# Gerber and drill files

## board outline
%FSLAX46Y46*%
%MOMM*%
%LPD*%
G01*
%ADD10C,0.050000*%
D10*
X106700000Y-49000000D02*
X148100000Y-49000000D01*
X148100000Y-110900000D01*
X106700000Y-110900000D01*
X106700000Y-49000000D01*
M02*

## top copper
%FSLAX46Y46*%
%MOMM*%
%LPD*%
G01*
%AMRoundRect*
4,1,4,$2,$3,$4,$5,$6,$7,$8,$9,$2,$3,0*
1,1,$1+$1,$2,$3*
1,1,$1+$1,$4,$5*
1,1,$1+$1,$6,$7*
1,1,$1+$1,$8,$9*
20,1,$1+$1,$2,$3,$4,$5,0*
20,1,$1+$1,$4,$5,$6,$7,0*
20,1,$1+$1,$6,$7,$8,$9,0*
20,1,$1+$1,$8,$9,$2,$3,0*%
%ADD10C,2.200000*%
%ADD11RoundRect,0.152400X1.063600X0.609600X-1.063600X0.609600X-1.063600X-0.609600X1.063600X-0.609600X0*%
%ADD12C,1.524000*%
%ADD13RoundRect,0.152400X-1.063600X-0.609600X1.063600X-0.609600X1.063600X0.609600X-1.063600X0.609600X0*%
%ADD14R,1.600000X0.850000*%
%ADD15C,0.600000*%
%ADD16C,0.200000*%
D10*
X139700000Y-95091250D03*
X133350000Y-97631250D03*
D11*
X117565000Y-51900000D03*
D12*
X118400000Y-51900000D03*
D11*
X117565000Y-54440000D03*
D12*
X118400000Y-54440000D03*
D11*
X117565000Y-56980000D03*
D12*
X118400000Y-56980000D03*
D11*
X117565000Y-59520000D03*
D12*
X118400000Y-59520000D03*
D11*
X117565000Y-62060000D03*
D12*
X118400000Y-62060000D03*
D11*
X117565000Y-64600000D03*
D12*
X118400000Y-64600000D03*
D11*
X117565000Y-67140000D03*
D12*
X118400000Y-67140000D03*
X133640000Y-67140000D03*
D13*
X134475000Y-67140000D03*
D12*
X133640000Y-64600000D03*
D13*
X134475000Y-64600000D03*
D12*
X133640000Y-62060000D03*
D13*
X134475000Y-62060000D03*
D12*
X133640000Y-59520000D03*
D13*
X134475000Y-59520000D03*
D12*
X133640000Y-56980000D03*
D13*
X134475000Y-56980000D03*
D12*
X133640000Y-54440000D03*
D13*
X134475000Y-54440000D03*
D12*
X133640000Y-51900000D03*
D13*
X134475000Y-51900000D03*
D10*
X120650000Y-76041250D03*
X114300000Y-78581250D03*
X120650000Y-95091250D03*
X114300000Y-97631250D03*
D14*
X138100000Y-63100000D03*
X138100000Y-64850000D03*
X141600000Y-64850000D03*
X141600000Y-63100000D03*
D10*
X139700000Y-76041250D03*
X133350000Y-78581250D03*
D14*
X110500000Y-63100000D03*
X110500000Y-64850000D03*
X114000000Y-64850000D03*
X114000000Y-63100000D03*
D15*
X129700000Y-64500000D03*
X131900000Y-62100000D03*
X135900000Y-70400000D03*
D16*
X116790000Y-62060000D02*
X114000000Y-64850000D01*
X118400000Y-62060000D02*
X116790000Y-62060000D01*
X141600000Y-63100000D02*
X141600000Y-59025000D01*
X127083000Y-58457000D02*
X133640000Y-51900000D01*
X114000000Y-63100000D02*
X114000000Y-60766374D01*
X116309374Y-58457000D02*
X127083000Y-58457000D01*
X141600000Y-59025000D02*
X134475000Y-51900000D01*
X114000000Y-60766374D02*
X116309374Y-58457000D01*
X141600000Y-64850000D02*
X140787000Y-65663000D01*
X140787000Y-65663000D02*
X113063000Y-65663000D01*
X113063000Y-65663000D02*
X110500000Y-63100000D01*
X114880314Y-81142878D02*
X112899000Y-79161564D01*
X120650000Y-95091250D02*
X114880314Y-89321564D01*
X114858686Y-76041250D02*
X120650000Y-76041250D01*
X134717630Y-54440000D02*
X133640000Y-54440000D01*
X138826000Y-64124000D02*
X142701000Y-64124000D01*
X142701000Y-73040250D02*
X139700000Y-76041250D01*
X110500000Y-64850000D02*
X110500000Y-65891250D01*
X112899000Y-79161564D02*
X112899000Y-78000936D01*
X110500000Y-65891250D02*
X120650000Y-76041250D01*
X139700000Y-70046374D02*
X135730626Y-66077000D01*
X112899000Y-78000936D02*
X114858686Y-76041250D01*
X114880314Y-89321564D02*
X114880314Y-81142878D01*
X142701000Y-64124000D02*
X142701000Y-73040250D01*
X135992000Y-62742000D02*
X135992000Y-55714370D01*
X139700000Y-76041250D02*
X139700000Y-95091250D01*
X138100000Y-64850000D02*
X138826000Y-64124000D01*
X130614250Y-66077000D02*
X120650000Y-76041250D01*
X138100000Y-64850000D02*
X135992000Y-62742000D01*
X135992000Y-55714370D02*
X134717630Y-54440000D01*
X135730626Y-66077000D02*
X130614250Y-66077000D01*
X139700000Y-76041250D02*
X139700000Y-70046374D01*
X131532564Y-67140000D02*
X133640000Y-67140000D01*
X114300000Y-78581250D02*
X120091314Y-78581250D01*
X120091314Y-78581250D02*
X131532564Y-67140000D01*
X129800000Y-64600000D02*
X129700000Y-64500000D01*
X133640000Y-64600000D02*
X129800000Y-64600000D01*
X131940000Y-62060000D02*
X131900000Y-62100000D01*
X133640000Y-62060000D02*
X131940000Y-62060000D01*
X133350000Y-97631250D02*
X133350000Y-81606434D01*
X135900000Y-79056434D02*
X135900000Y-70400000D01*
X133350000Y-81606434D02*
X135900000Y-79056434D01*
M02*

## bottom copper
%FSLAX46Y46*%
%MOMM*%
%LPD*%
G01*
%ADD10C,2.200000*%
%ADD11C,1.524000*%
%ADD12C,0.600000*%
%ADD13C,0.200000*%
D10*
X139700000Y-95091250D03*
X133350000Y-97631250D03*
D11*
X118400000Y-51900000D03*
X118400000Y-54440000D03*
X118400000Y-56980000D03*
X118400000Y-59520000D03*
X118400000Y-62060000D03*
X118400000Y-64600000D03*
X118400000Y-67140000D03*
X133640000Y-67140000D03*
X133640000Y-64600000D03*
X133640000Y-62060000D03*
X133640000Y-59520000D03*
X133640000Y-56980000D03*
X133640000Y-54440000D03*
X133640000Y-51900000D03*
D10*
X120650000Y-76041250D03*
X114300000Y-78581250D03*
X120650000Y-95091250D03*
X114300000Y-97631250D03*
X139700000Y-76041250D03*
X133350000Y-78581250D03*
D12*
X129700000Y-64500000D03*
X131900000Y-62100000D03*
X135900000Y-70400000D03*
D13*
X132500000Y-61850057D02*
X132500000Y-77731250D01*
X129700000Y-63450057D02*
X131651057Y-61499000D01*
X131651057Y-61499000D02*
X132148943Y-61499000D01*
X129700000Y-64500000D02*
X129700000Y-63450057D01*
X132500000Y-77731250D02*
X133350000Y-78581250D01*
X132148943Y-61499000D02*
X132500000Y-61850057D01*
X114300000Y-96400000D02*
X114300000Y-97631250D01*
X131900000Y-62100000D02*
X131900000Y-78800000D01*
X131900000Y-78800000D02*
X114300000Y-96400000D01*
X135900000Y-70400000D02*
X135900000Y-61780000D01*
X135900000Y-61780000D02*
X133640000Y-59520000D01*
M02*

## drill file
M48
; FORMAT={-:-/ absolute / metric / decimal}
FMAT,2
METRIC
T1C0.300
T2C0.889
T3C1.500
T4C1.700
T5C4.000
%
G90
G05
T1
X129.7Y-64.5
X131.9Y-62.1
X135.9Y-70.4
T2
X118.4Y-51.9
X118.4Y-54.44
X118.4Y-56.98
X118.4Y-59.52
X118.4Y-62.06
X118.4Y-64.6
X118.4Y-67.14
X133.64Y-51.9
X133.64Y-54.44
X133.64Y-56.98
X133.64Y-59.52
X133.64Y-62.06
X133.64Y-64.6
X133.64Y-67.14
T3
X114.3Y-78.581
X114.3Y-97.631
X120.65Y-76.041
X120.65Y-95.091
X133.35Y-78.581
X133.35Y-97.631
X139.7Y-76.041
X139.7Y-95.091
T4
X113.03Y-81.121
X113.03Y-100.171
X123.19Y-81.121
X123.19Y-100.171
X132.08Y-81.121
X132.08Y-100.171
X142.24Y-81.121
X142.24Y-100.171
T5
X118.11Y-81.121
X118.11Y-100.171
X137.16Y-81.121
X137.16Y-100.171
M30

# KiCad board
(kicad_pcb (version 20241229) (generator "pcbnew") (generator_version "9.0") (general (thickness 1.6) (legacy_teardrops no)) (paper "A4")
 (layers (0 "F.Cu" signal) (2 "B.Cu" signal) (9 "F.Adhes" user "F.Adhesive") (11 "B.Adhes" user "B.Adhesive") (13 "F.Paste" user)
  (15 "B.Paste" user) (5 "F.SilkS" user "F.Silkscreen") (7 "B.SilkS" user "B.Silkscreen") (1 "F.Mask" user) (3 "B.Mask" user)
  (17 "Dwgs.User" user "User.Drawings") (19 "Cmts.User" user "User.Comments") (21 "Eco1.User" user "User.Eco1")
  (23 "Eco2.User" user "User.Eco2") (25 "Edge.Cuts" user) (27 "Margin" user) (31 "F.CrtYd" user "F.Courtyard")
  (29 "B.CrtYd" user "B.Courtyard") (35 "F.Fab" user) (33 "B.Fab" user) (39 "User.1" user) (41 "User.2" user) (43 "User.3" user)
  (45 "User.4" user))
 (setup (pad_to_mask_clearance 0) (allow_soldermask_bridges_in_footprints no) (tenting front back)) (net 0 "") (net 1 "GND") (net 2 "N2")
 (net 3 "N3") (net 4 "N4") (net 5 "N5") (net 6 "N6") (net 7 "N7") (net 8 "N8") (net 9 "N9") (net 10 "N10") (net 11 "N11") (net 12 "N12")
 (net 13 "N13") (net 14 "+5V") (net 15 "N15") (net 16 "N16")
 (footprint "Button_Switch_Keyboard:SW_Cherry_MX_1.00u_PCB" (layer "F.Cu") (at 139.7 95.09125)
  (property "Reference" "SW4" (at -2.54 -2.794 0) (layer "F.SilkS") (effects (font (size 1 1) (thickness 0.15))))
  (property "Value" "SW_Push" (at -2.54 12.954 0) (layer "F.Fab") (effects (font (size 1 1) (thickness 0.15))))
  (pad "" np_thru_hole circle (at -7.62 5.08) (size 1.7 1.7) (drill 1.7) (layers "*.Cu" "*.Mask"))
  (pad "" np_thru_hole circle (at -2.54 5.08) (size 4 4) (drill 4) (layers "*.Cu" "*.Mask"))
  (pad "" np_thru_hole circle (at 2.54 5.08) (size 1.7 1.7) (drill 1.7) (layers "*.Cu" "*.Mask"))
  (pad "1" thru_hole circle (at 0 0) (size 2.2 2.2) (drill 1.5) (layers "*.Cu" "*.Mask") (remove_unused_layers no) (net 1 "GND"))
  (pad "2" thru_hole circle (at -6.35 2.54) (size 2.2 2.2) (drill 1.5) (layers "*.Cu" "*.Mask") (remove_unused_layers no) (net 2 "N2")))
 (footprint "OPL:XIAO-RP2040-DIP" (layer "F.Cu") (at 126.02 59.52)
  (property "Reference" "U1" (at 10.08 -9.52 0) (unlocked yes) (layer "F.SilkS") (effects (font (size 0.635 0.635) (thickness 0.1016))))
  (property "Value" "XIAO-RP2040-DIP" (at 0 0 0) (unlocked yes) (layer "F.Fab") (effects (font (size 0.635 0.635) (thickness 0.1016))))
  (pad "1" smd roundrect (at -8.455 -7.62 180) (size 2.432 1.524) (layers "F.Cu" "F.Mask") (roundrect_rratio 0.1) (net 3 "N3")
   (thermal_bridge_angle 45))
  (pad "1" thru_hole circle (at -7.62 -7.62 180) (size 1.524 1.524) (drill 0.889) (layers "*.Cu" "*.Mask") (remove_unused_layers no)
   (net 3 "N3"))
  (pad "2" smd roundrect (at -8.455 -5.08 180) (size 2.432 1.524) (layers "F.Cu" "F.Mask") (roundrect_rratio 0.1) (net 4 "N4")
   (thermal_bridge_angle 45))
  (pad "2" thru_hole circle (at -7.62 -5.08 180) (size 1.524 1.524) (drill 0.889) (layers "*.Cu" "*.Mask") (remove_unused_layers no)
   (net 4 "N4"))
  (pad "3" smd roundrect (at -8.455 -2.54 180) (size 2.432 1.524) (layers "F.Cu" "F.Mask") (roundrect_rratio 0.1) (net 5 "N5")
   (thermal_bridge_angle 45))
  (pad "3" thru_hole circle (at -7.62 -2.54 180) (size 1.524 1.524) (drill 0.889) (layers "*.Cu" "*.Mask") (remove_unused_layers no)
   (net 5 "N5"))
  (pad "4" smd roundrect (at -8.455 0 180) (size 2.432 1.524) (layers "F.Cu" "F.Mask") (roundrect_rratio 0.1) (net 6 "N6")
   (thermal_bridge_angle 45))
  (pad "4" thru_hole circle (at -7.62 0 180) (size 1.524 1.524) (drill 0.889) (layers "*.Cu" "*.Mask") (remove_unused_layers no)
   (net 6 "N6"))
  (pad "5" smd roundrect (at -8.455 2.54 180) (size 2.432 1.524) (layers "F.Cu" "F.Mask") (roundrect_rratio 0.1) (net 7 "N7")
   (thermal_bridge_angle 45))
  (pad "5" thru_hole circle (at -7.62 2.54 180) (size 1.524 1.524) (drill 0.889) (layers "*.Cu" "*.Mask") (remove_unused_layers no)
   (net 7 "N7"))
  (pad "6" smd roundrect (at -8.455 5.08 180) (size 2.432 1.524) (layers "F.Cu" "F.Mask") (roundrect_rratio 0.1) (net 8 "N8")
   (thermal_bridge_angle 45))
  (pad "6" thru_hole circle (at -7.62 5.08 180) (size 1.524 1.524) (drill 0.889) (layers "*.Cu" "*.Mask") (remove_unused_layers no)
   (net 8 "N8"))
  (pad "7" smd roundrect (at -8.455 7.62 180) (size 2.432 1.524) (layers "F.Cu" "F.Mask") (roundrect_rratio 0.1) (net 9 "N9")
   (thermal_bridge_angle 45))
  (pad "7" thru_hole circle (at -7.62 7.62 180) (size 1.524 1.524) (drill 0.889) (layers "*.Cu" "*.Mask") (remove_unused_layers no)
   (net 9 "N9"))
  (pad "8" thru_hole circle (at 7.62 7.62) (size 1.524 1.524) (drill 0.889) (layers "*.Cu" "*.Mask") (remove_unused_layers no)
   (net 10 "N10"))
  (pad "8" smd roundrect (at 8.455 7.62) (size 2.432 1.524) (layers "F.Cu" "F.Mask") (roundrect_rratio 0.1) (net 10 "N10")
   (thermal_bridge_angle 45))
  (pad "9" thru_hole circle (at 7.62 5.08) (size 1.524 1.524) (drill 0.889) (layers "*.Cu" "*.Mask") (remove_unused_layers no)
   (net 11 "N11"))
  (pad "9" smd roundrect (at 8.455 5.08) (size 2.432 1.524) (layers "F.Cu" "F.Mask") (roundrect_rratio 0.1) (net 11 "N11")
   (thermal_bridge_angle 45))
  (pad "10" thru_hole circle (at 7.62 2.54) (size 1.524 1.524) (drill 0.889) (layers "*.Cu" "*.Mask") (remove_unused_layers no)
   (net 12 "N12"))
  (pad "10" smd roundrect (at 8.455 2.54) (size 2.432 1.524) (layers "F.Cu" "F.Mask") (roundrect_rratio 0.1) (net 12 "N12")
   (thermal_bridge_angle 45))
  (pad "11" thru_hole circle (at 7.62 0) (size 1.524 1.524) (drill 0.889) (layers "*.Cu" "*.Mask") (remove_unused_layers no) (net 2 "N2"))
  (pad "11" smd roundrect (at 8.455 0) (size 2.432 1.524) (layers "F.Cu" "F.Mask") (roundrect_rratio 0.1) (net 2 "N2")
   (thermal_bridge_angle 45))
  (pad "12" thru_hole circle (at 7.62 -2.54) (size 1.524 1.524) (drill 0.889) (layers "*.Cu" "*.Mask") (remove_unused_layers no)
   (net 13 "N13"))
  (pad "12" smd roundrect (at 8.455 -2.54) (size 2.432 1.524) (layers "F.Cu" "F.Mask") (roundrect_rratio 0.1) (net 13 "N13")
   (thermal_bridge_angle 45))
  (pad "13" thru_hole circle (at 7.62 -5.08) (size 1.524 1.524) (drill 0.889) (layers "*.Cu" "*.Mask") (remove_unused_layers no)
   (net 1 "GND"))
  (pad "13" smd roundrect (at 8.455 -5.08) (size 2.432 1.524) (layers "F.Cu" "F.Mask") (roundrect_rratio 0.1) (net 1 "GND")
   (thermal_bridge_angle 45))
  (pad "14" thru_hole circle (at 7.62 -7.62) (size 1.524 1.524) (drill 0.889) (layers "*.Cu" "*.Mask") (remove_unused_layers no)
   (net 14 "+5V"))
  (pad "14" smd roundrect (at 8.455 -7.62) (size 2.432 1.524) (layers "F.Cu" "F.Mask") (roundrect_rratio 0.1) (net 14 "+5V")
   (thermal_bridge_angle 45)))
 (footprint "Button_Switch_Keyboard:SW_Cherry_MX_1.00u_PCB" (layer "F.Cu") (at 120.65 76.04125)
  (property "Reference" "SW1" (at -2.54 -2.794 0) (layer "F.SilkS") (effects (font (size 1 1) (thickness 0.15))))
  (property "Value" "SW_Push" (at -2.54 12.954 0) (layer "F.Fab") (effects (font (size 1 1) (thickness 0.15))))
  (pad "" np_thru_hole circle (at -7.62 5.08) (size 1.7 1.7) (drill 1.7) (layers "*.Cu" "*.Mask"))
  (pad "" np_thru_hole circle (at -2.54 5.08) (size 4 4) (drill 4) (layers "*.Cu" "*.Mask"))
  (pad "" np_thru_hole circle (at 2.54 5.08) (size 1.7 1.7) (drill 1.7) (layers "*.Cu" "*.Mask"))
  (pad "1" thru_hole circle (at 0 0) (size 2.2 2.2) (drill 1.5) (layers "*.Cu" "*.Mask") (remove_unused_layers no) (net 1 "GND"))
  (pad "2" thru_hole circle (at -6.35 2.54) (size 2.2 2.2) (drill 1.5) (layers "*.Cu" "*.Mask") (remove_unused_layers no) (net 10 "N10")))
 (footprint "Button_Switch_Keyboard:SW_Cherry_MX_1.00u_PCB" (layer "F.Cu") (at 120.65 95.09125)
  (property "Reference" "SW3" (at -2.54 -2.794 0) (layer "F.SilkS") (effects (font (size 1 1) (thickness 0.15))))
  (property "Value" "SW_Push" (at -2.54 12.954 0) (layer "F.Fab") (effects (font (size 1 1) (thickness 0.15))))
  (pad "" np_thru_hole circle (at -7.62 5.08) (size 1.7 1.7) (drill 1.7) (layers "*.Cu" "*.Mask"))
  (pad "" np_thru_hole circle (at -2.54 5.08) (size 4 4) (drill 4) (layers "*.Cu" "*.Mask"))
  (pad "" np_thru_hole circle (at 2.54 5.08) (size 1.7 1.7) (drill 1.7) (layers "*.Cu" "*.Mask"))
  (pad "1" thru_hole circle (at 0 0) (size 2.2 2.2) (drill 1.5) (layers "*.Cu" "*.Mask") (remove_unused_layers no) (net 1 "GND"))
  (pad "2" thru_hole circle (at -6.35 2.54) (size 2.2 2.2) (drill 1.5) (layers "*.Cu" "*.Mask") (remove_unused_layers no) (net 12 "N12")))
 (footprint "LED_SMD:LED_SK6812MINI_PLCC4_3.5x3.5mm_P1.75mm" (layer "F.Cu") (at 139.85 63.975)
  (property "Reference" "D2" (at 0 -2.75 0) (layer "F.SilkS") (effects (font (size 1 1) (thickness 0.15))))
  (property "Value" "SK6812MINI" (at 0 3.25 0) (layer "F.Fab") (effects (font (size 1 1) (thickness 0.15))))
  (pad "1" smd rect (at -1.75 -0.875) (size 1.6 0.85) (layers "F.Cu" "F.Mask" "F.Paste") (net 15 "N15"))
  (pad "2" smd rect (at -1.75 0.875) (size 1.6 0.85) (layers "F.Cu" "F.Mask" "F.Paste") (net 1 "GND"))
  (pad "3" smd rect (at 1.75 0.875) (size 1.6 0.85) (layers "F.Cu" "F.Mask" "F.Paste") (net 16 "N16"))
  (pad "4" smd rect (at 1.75 -0.875) (size 1.6 0.85) (layers "F.Cu" "F.Mask" "F.Paste") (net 14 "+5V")))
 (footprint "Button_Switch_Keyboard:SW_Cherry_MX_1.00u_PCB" (layer "F.Cu") (at 139.7 76.04125)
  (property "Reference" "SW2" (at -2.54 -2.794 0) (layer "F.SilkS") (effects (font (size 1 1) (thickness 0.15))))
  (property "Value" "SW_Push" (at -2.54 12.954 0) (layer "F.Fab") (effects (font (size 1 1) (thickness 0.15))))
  (pad "" np_thru_hole circle (at -7.62 5.08) (size 1.7 1.7) (drill 1.7) (layers "*.Cu" "*.Mask"))
  (pad "" np_thru_hole circle (at -2.54 5.08) (size 4 4) (drill 4) (layers "*.Cu" "*.Mask"))
  (pad "" np_thru_hole circle (at 2.54 5.08) (size 1.7 1.7) (drill 1.7) (layers "*.Cu" "*.Mask"))
  (pad "1" thru_hole circle (at 0 0) (size 2.2 2.2) (drill 1.5) (layers "*.Cu" "*.Mask") (remove_unused_layers no) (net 1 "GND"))
  (pad "2" thru_hole circle (at -6.35 2.54) (size 2.2 2.2) (drill 1.5) (layers "*.Cu" "*.Mask") (remove_unused_layers no) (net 11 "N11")))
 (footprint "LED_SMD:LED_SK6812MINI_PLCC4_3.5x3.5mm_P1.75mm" (layer "F.Cu") (at 112.25 63.975)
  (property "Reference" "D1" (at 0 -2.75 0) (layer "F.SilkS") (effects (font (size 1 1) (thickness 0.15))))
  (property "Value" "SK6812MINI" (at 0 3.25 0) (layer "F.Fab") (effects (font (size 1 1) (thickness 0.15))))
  (pad "1" smd rect (at -1.75 -0.875) (size 1.6 0.85) (layers "F.Cu" "F.Mask" "F.Paste") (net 16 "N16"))
  (pad "2" smd rect (at -1.75 0.875) (size 1.6 0.85) (layers "F.Cu" "F.Mask" "F.Paste") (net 1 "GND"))
  (pad "3" smd rect (at 1.75 0.875) (size 1.6 0.85) (layers "F.Cu" "F.Mask" "F.Paste") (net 7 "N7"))
  (pad "4" smd rect (at 1.75 -0.875) (size 1.6 0.85) (layers "F.Cu" "F.Mask" "F.Paste") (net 14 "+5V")))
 (gr_rect (start 106.7 49) (end 148.1 110.9) (stroke (width 0.05) (type default)) (fill no) (layer "Edge.Cuts"))
 (segment (start 116.79 62.06) (end 114 64.85) (width 0.2) (layer "F.Cu") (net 7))
 (segment (start 118.4 62.06) (end 116.79 62.06) (width 0.2) (layer "F.Cu") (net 7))
 (segment (start 141.6 63.1) (end 141.6 59.025) (width 0.2) (layer "F.Cu") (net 14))
 (segment (start 127.083 58.457) (end 133.64 51.9) (width 0.2) (layer "F.Cu") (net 14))
 (segment (start 114 63.1) (end 114 60.766374) (width 0.2) (layer "F.Cu") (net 14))
 (segment (start 116.309374 58.457) (end 127.083 58.457) (width 0.2) (layer "F.Cu") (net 14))
 (segment (start 141.6 59.025) (end 134.475 51.9) (width 0.2) (layer "F.Cu") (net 14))
 (segment (start 114 60.766374) (end 116.309374 58.457) (width 0.2) (layer "F.Cu") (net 14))
 (segment (start 141.6 64.85) (end 140.787 65.663) (width 0.2) (layer "F.Cu") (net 16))
 (segment (start 140.787 65.663) (end 113.063 65.663) (width 0.2) (layer "F.Cu") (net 16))
 (segment (start 113.063 65.663) (end 110.5 63.1) (width 0.2) (layer "F.Cu") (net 16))
 (segment (start 114.880314 81.142878) (end 112.899 79.161564) (width 0.2) (layer "F.Cu") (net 1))
 (segment (start 120.65 95.09125) (end 114.880314 89.321564) (width 0.2) (layer "F.Cu") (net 1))
 (segment (start 114.858686 76.04125) (end 120.65 76.04125) (width 0.2) (layer "F.Cu") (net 1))
 (segment (start 134.71763 54.44) (end 133.64 54.44) (width 0.2) (layer "F.Cu") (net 1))
 (segment (start 138.826 64.124) (end 142.701 64.124) (width 0.2) (layer "F.Cu") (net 1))
 (segment (start 142.701 73.04025) (end 139.7 76.04125) (width 0.2) (layer "F.Cu") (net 1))
 (segment (start 110.5 64.85) (end 110.5 65.89125) (width 0.2) (layer "F.Cu") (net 1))
 (segment (start 112.899 79.161564) (end 112.899 78.000936) (width 0.2) (layer "F.Cu") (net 1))
 (segment (start 110.5 65.89125) (end 120.65 76.04125) (width 0.2) (layer "F.Cu") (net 1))
 (segment (start 139.7 70.046374) (end 135.730626 66.077) (width 0.2) (layer "F.Cu") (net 1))
 (segment (start 112.899 78.000936) (end 114.858686 76.04125) (width 0.2) (layer "F.Cu") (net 1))
 (segment (start 114.880314 89.321564) (end 114.880314 81.142878) (width 0.2) (layer "F.Cu") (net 1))
 (segment (start 142.701 64.124) (end 142.701 73.04025) (width 0.2) (layer "F.Cu") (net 1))
 (segment (start 135.992 62.742) (end 135.992 55.71437) (width 0.2) (layer "F.Cu") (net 1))
 (segment (start 139.7 76.04125) (end 139.7 95.09125) (width 0.2) (layer "F.Cu") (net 1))
 (segment (start 138.1 64.85) (end 138.826 64.124) (width 0.2) (layer "F.Cu") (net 1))
 (segment (start 130.61425 66.077) (end 120.65 76.04125) (width 0.2) (layer "F.Cu") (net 1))
 (segment (start 138.1 64.85) (end 135.992 62.742) (width 0.2) (layer "F.Cu") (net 1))
 (segment (start 135.992 55.71437) (end 134.71763 54.44) (width 0.2) (layer "F.Cu") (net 1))
 (segment (start 135.730626 66.077) (end 130.61425 66.077) (width 0.2) (layer "F.Cu") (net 1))
 (segment (start 139.7 76.04125) (end 139.7 70.046374) (width 0.2) (layer "F.Cu") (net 1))
 (segment (start 131.532564 67.14) (end 133.64 67.14) (width 0.2) (layer "F.Cu") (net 10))
 (segment (start 114.3 78.58125) (end 120.091314 78.58125) (width 0.2) (layer "F.Cu") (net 10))
 (segment (start 120.091314 78.58125) (end 131.532564 67.14) (width 0.2) (layer "F.Cu") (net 10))
 (segment (start 129.8 64.6) (end 129.7 64.5) (width 0.2) (layer "F.Cu") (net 11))
 (segment (start 133.64 64.6) (end 129.8 64.6) (width 0.2) (layer "F.Cu") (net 11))
 (via (at 129.7 64.5) (size 0.6) (drill 0.3) (layers "F.Cu" "B.Cu") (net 11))
 (segment (start 132.5 61.850057) (end 132.5 77.73125) (width 0.2) (layer "B.Cu") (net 11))
 (segment (start 129.7 63.450057) (end 131.651057 61.499) (width 0.2) (layer "B.Cu") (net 11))
 (segment (start 131.651057 61.499) (end 132.148943 61.499) (width 0.2) (layer "B.Cu") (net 11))
 (segment (start 129.7 64.5) (end 129.7 63.450057) (width 0.2) (layer "B.Cu") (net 11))
 (segment (start 132.5 77.73125) (end 133.35 78.58125) (width 0.2) (layer "B.Cu") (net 11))
 (segment (start 132.148943 61.499) (end 132.5 61.850057) (width 0.2) (layer "B.Cu") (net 11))
 (segment (start 131.94 62.06) (end 131.9 62.1) (width 0.2) (layer "F.Cu") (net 12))
 (segment (start 133.64 62.06) (end 131.94 62.06) (width 0.2) (layer "F.Cu") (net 12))
 (via (at 131.9 62.1) (size 0.6) (drill 0.3) (layers "F.Cu" "B.Cu") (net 12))
 (segment (start 114.3 96.4) (end 114.3 97.63125) (width 0.2) (layer "B.Cu") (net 12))
 (segment (start 131.9 62.1) (end 131.9 78.8) (width 0.2) (layer "B.Cu") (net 12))
 (segment (start 131.9 78.8) (end 114.3 96.4) (width 0.2) (layer "B.Cu") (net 12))
 (segment (start 133.35 97.63125) (end 133.35 81.606434) (width 0.2) (layer "F.Cu") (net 2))
 (segment (start 135.9 79.056434) (end 135.9 70.4) (width 0.2) (layer "F.Cu") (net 2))
 (segment (start 133.35 81.606434) (end 135.9 79.056434) (width 0.2) (layer "F.Cu") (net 2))
 (via (at 135.9 70.4) (size 0.6) (drill 0.3) (layers "F.Cu" "B.Cu") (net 2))
 (segment (start 135.9 70.4) (end 135.9 61.78) (width 0.2) (layer "B.Cu") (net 2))
 (segment (start 135.9 61.78) (end 133.64 59.52) (width 0.2) (layer "B.Cu") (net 2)))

